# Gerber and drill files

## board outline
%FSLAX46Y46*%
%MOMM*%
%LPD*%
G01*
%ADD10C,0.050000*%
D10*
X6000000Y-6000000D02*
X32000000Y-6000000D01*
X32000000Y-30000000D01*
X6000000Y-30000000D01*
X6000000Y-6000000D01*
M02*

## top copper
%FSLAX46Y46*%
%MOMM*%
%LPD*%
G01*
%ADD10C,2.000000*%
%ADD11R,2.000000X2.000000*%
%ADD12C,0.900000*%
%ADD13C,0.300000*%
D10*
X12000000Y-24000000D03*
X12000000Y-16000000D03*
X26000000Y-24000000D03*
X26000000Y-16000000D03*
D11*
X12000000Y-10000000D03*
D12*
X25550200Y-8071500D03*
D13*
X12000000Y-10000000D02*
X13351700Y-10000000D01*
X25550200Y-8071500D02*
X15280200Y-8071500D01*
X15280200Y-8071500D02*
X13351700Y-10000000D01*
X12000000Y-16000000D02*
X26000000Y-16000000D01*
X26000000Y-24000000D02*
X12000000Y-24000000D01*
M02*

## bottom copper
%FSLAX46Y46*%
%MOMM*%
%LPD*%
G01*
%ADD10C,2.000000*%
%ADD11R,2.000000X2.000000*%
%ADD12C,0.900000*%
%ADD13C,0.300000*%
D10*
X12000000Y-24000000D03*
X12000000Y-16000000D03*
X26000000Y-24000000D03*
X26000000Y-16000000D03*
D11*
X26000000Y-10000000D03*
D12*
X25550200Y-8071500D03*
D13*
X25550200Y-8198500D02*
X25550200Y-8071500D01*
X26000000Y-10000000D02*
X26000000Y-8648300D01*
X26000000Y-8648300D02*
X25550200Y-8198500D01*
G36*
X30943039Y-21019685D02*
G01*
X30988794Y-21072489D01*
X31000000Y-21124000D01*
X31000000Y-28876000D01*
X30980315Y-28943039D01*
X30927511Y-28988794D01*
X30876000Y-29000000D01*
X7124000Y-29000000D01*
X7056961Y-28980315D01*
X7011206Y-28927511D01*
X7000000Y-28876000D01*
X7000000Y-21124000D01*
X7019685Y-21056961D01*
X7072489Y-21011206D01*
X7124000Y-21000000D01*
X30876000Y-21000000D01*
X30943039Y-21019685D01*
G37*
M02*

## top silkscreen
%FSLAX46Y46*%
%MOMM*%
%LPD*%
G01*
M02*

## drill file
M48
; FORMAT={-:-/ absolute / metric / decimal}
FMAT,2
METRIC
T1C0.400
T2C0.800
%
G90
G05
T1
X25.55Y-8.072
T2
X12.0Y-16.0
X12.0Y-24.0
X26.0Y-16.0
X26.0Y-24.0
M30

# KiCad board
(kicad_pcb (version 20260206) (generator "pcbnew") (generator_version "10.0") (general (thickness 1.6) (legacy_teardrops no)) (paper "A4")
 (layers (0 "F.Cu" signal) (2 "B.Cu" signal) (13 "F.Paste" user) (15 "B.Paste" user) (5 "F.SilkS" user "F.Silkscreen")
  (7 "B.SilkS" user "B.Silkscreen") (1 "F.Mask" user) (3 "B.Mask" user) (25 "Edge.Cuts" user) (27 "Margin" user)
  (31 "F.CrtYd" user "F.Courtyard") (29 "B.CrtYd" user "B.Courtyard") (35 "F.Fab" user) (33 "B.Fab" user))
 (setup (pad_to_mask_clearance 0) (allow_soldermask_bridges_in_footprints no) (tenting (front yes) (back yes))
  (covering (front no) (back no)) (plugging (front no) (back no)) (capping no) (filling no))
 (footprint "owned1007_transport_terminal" (layer "F.Cu") (at 12 24)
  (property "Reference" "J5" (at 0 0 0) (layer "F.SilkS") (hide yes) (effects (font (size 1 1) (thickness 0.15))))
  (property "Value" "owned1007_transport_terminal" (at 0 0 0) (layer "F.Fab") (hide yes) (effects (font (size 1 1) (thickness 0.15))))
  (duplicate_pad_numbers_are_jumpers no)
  (pad "1" thru_hole circle (at 0 0) (size 2 2) (drill 0.8) (layers "*.Cu" "*.Mask") (remove_unused_layers no) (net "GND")))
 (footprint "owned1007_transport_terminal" (layer "F.Cu") (at 12 16)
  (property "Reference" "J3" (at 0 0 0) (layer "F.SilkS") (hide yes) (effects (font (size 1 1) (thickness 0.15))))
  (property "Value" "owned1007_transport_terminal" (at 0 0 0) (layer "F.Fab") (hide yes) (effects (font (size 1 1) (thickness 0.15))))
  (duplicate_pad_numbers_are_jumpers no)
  (pad "1" thru_hole circle (at 0 0) (size 2 2) (drill 0.8) (layers "*.Cu" "*.Mask") (remove_unused_layers no) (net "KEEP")))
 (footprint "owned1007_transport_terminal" (layer "F.Cu") (at 26 24)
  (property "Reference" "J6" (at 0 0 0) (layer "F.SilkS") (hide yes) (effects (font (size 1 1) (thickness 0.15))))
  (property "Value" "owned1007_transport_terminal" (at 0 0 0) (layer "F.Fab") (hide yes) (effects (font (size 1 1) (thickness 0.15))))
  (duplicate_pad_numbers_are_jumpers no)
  (pad "1" thru_hole circle (at 0 0) (size 2 2) (drill 0.8) (layers "*.Cu" "*.Mask") (remove_unused_layers no) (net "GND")))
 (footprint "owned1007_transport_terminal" (layer "F.Cu") (at 26 16)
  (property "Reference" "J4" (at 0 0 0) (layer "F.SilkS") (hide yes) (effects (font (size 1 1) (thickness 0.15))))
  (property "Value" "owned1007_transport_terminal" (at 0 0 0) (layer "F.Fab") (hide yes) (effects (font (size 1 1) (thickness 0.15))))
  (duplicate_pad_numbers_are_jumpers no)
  (pad "1" thru_hole circle (at 0 0) (size 2 2) (drill 0.8) (layers "*.Cu" "*.Mask") (remove_unused_layers no) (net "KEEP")))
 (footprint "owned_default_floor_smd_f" (layer "F.Cu") (at 12 10)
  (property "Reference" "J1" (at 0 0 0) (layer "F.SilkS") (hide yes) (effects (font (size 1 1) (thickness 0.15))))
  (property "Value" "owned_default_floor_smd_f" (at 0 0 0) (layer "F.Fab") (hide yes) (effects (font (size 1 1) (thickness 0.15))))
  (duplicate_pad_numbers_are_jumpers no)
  (pad "1" smd rect (at 0 0) (size 2 2) (layers "F.Cu" "F.Mask" "F.Paste") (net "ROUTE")))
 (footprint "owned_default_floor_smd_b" (layer "B.Cu") (at 26 10)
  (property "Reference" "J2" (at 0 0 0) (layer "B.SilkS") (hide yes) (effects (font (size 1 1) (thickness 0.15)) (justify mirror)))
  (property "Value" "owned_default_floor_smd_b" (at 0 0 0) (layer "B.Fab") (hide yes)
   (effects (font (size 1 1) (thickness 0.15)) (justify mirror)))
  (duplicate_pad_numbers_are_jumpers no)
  (pad "1" smd rect (at 0 0) (size 2 2) (layers "B.Cu" "B.Mask" "B.Paste") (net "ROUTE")))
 (gr_rect (start 6 6) (end 32 30) (stroke (width 0.05) (type default)) (fill no) (layer "Edge.Cuts"))
 (segment (start 12 10) (end 13.3517 10) (width 0.3) (layer "F.Cu") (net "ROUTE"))
 (segment (start 25.5502 8.0715) (end 15.2802 8.0715) (width 0.3) (layer "F.Cu") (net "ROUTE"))
 (segment (start 15.2802 8.0715) (end 13.3517 10) (width 0.3) (layer "F.Cu") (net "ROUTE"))
 (via (at 25.5502 8.0715) (size 0.9) (drill 0.4) (layers "F.Cu" "B.Cu") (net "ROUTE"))
 (segment (start 25.5502 8.1985) (end 25.5502 8.0715) (width 0.3) (layer "B.Cu") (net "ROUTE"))
 (segment (start 26 10) (end 26 8.6483) (width 0.3) (layer "B.Cu") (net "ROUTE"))
 (segment (start 26 8.6483) (end 25.5502 8.1985) (width 0.3) (layer "B.Cu") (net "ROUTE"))
 (segment (start 12 16) (end 26 16) (width 0.3) (locked yes) (layer "F.Cu") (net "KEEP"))
 (segment (start 26 24) (end 12 24) (width 0.3) (layer "F.Cu") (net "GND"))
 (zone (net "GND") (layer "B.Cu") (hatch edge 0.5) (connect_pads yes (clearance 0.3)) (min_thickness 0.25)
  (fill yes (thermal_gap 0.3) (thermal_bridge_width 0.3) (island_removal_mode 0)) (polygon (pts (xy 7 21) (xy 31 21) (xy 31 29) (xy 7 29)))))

